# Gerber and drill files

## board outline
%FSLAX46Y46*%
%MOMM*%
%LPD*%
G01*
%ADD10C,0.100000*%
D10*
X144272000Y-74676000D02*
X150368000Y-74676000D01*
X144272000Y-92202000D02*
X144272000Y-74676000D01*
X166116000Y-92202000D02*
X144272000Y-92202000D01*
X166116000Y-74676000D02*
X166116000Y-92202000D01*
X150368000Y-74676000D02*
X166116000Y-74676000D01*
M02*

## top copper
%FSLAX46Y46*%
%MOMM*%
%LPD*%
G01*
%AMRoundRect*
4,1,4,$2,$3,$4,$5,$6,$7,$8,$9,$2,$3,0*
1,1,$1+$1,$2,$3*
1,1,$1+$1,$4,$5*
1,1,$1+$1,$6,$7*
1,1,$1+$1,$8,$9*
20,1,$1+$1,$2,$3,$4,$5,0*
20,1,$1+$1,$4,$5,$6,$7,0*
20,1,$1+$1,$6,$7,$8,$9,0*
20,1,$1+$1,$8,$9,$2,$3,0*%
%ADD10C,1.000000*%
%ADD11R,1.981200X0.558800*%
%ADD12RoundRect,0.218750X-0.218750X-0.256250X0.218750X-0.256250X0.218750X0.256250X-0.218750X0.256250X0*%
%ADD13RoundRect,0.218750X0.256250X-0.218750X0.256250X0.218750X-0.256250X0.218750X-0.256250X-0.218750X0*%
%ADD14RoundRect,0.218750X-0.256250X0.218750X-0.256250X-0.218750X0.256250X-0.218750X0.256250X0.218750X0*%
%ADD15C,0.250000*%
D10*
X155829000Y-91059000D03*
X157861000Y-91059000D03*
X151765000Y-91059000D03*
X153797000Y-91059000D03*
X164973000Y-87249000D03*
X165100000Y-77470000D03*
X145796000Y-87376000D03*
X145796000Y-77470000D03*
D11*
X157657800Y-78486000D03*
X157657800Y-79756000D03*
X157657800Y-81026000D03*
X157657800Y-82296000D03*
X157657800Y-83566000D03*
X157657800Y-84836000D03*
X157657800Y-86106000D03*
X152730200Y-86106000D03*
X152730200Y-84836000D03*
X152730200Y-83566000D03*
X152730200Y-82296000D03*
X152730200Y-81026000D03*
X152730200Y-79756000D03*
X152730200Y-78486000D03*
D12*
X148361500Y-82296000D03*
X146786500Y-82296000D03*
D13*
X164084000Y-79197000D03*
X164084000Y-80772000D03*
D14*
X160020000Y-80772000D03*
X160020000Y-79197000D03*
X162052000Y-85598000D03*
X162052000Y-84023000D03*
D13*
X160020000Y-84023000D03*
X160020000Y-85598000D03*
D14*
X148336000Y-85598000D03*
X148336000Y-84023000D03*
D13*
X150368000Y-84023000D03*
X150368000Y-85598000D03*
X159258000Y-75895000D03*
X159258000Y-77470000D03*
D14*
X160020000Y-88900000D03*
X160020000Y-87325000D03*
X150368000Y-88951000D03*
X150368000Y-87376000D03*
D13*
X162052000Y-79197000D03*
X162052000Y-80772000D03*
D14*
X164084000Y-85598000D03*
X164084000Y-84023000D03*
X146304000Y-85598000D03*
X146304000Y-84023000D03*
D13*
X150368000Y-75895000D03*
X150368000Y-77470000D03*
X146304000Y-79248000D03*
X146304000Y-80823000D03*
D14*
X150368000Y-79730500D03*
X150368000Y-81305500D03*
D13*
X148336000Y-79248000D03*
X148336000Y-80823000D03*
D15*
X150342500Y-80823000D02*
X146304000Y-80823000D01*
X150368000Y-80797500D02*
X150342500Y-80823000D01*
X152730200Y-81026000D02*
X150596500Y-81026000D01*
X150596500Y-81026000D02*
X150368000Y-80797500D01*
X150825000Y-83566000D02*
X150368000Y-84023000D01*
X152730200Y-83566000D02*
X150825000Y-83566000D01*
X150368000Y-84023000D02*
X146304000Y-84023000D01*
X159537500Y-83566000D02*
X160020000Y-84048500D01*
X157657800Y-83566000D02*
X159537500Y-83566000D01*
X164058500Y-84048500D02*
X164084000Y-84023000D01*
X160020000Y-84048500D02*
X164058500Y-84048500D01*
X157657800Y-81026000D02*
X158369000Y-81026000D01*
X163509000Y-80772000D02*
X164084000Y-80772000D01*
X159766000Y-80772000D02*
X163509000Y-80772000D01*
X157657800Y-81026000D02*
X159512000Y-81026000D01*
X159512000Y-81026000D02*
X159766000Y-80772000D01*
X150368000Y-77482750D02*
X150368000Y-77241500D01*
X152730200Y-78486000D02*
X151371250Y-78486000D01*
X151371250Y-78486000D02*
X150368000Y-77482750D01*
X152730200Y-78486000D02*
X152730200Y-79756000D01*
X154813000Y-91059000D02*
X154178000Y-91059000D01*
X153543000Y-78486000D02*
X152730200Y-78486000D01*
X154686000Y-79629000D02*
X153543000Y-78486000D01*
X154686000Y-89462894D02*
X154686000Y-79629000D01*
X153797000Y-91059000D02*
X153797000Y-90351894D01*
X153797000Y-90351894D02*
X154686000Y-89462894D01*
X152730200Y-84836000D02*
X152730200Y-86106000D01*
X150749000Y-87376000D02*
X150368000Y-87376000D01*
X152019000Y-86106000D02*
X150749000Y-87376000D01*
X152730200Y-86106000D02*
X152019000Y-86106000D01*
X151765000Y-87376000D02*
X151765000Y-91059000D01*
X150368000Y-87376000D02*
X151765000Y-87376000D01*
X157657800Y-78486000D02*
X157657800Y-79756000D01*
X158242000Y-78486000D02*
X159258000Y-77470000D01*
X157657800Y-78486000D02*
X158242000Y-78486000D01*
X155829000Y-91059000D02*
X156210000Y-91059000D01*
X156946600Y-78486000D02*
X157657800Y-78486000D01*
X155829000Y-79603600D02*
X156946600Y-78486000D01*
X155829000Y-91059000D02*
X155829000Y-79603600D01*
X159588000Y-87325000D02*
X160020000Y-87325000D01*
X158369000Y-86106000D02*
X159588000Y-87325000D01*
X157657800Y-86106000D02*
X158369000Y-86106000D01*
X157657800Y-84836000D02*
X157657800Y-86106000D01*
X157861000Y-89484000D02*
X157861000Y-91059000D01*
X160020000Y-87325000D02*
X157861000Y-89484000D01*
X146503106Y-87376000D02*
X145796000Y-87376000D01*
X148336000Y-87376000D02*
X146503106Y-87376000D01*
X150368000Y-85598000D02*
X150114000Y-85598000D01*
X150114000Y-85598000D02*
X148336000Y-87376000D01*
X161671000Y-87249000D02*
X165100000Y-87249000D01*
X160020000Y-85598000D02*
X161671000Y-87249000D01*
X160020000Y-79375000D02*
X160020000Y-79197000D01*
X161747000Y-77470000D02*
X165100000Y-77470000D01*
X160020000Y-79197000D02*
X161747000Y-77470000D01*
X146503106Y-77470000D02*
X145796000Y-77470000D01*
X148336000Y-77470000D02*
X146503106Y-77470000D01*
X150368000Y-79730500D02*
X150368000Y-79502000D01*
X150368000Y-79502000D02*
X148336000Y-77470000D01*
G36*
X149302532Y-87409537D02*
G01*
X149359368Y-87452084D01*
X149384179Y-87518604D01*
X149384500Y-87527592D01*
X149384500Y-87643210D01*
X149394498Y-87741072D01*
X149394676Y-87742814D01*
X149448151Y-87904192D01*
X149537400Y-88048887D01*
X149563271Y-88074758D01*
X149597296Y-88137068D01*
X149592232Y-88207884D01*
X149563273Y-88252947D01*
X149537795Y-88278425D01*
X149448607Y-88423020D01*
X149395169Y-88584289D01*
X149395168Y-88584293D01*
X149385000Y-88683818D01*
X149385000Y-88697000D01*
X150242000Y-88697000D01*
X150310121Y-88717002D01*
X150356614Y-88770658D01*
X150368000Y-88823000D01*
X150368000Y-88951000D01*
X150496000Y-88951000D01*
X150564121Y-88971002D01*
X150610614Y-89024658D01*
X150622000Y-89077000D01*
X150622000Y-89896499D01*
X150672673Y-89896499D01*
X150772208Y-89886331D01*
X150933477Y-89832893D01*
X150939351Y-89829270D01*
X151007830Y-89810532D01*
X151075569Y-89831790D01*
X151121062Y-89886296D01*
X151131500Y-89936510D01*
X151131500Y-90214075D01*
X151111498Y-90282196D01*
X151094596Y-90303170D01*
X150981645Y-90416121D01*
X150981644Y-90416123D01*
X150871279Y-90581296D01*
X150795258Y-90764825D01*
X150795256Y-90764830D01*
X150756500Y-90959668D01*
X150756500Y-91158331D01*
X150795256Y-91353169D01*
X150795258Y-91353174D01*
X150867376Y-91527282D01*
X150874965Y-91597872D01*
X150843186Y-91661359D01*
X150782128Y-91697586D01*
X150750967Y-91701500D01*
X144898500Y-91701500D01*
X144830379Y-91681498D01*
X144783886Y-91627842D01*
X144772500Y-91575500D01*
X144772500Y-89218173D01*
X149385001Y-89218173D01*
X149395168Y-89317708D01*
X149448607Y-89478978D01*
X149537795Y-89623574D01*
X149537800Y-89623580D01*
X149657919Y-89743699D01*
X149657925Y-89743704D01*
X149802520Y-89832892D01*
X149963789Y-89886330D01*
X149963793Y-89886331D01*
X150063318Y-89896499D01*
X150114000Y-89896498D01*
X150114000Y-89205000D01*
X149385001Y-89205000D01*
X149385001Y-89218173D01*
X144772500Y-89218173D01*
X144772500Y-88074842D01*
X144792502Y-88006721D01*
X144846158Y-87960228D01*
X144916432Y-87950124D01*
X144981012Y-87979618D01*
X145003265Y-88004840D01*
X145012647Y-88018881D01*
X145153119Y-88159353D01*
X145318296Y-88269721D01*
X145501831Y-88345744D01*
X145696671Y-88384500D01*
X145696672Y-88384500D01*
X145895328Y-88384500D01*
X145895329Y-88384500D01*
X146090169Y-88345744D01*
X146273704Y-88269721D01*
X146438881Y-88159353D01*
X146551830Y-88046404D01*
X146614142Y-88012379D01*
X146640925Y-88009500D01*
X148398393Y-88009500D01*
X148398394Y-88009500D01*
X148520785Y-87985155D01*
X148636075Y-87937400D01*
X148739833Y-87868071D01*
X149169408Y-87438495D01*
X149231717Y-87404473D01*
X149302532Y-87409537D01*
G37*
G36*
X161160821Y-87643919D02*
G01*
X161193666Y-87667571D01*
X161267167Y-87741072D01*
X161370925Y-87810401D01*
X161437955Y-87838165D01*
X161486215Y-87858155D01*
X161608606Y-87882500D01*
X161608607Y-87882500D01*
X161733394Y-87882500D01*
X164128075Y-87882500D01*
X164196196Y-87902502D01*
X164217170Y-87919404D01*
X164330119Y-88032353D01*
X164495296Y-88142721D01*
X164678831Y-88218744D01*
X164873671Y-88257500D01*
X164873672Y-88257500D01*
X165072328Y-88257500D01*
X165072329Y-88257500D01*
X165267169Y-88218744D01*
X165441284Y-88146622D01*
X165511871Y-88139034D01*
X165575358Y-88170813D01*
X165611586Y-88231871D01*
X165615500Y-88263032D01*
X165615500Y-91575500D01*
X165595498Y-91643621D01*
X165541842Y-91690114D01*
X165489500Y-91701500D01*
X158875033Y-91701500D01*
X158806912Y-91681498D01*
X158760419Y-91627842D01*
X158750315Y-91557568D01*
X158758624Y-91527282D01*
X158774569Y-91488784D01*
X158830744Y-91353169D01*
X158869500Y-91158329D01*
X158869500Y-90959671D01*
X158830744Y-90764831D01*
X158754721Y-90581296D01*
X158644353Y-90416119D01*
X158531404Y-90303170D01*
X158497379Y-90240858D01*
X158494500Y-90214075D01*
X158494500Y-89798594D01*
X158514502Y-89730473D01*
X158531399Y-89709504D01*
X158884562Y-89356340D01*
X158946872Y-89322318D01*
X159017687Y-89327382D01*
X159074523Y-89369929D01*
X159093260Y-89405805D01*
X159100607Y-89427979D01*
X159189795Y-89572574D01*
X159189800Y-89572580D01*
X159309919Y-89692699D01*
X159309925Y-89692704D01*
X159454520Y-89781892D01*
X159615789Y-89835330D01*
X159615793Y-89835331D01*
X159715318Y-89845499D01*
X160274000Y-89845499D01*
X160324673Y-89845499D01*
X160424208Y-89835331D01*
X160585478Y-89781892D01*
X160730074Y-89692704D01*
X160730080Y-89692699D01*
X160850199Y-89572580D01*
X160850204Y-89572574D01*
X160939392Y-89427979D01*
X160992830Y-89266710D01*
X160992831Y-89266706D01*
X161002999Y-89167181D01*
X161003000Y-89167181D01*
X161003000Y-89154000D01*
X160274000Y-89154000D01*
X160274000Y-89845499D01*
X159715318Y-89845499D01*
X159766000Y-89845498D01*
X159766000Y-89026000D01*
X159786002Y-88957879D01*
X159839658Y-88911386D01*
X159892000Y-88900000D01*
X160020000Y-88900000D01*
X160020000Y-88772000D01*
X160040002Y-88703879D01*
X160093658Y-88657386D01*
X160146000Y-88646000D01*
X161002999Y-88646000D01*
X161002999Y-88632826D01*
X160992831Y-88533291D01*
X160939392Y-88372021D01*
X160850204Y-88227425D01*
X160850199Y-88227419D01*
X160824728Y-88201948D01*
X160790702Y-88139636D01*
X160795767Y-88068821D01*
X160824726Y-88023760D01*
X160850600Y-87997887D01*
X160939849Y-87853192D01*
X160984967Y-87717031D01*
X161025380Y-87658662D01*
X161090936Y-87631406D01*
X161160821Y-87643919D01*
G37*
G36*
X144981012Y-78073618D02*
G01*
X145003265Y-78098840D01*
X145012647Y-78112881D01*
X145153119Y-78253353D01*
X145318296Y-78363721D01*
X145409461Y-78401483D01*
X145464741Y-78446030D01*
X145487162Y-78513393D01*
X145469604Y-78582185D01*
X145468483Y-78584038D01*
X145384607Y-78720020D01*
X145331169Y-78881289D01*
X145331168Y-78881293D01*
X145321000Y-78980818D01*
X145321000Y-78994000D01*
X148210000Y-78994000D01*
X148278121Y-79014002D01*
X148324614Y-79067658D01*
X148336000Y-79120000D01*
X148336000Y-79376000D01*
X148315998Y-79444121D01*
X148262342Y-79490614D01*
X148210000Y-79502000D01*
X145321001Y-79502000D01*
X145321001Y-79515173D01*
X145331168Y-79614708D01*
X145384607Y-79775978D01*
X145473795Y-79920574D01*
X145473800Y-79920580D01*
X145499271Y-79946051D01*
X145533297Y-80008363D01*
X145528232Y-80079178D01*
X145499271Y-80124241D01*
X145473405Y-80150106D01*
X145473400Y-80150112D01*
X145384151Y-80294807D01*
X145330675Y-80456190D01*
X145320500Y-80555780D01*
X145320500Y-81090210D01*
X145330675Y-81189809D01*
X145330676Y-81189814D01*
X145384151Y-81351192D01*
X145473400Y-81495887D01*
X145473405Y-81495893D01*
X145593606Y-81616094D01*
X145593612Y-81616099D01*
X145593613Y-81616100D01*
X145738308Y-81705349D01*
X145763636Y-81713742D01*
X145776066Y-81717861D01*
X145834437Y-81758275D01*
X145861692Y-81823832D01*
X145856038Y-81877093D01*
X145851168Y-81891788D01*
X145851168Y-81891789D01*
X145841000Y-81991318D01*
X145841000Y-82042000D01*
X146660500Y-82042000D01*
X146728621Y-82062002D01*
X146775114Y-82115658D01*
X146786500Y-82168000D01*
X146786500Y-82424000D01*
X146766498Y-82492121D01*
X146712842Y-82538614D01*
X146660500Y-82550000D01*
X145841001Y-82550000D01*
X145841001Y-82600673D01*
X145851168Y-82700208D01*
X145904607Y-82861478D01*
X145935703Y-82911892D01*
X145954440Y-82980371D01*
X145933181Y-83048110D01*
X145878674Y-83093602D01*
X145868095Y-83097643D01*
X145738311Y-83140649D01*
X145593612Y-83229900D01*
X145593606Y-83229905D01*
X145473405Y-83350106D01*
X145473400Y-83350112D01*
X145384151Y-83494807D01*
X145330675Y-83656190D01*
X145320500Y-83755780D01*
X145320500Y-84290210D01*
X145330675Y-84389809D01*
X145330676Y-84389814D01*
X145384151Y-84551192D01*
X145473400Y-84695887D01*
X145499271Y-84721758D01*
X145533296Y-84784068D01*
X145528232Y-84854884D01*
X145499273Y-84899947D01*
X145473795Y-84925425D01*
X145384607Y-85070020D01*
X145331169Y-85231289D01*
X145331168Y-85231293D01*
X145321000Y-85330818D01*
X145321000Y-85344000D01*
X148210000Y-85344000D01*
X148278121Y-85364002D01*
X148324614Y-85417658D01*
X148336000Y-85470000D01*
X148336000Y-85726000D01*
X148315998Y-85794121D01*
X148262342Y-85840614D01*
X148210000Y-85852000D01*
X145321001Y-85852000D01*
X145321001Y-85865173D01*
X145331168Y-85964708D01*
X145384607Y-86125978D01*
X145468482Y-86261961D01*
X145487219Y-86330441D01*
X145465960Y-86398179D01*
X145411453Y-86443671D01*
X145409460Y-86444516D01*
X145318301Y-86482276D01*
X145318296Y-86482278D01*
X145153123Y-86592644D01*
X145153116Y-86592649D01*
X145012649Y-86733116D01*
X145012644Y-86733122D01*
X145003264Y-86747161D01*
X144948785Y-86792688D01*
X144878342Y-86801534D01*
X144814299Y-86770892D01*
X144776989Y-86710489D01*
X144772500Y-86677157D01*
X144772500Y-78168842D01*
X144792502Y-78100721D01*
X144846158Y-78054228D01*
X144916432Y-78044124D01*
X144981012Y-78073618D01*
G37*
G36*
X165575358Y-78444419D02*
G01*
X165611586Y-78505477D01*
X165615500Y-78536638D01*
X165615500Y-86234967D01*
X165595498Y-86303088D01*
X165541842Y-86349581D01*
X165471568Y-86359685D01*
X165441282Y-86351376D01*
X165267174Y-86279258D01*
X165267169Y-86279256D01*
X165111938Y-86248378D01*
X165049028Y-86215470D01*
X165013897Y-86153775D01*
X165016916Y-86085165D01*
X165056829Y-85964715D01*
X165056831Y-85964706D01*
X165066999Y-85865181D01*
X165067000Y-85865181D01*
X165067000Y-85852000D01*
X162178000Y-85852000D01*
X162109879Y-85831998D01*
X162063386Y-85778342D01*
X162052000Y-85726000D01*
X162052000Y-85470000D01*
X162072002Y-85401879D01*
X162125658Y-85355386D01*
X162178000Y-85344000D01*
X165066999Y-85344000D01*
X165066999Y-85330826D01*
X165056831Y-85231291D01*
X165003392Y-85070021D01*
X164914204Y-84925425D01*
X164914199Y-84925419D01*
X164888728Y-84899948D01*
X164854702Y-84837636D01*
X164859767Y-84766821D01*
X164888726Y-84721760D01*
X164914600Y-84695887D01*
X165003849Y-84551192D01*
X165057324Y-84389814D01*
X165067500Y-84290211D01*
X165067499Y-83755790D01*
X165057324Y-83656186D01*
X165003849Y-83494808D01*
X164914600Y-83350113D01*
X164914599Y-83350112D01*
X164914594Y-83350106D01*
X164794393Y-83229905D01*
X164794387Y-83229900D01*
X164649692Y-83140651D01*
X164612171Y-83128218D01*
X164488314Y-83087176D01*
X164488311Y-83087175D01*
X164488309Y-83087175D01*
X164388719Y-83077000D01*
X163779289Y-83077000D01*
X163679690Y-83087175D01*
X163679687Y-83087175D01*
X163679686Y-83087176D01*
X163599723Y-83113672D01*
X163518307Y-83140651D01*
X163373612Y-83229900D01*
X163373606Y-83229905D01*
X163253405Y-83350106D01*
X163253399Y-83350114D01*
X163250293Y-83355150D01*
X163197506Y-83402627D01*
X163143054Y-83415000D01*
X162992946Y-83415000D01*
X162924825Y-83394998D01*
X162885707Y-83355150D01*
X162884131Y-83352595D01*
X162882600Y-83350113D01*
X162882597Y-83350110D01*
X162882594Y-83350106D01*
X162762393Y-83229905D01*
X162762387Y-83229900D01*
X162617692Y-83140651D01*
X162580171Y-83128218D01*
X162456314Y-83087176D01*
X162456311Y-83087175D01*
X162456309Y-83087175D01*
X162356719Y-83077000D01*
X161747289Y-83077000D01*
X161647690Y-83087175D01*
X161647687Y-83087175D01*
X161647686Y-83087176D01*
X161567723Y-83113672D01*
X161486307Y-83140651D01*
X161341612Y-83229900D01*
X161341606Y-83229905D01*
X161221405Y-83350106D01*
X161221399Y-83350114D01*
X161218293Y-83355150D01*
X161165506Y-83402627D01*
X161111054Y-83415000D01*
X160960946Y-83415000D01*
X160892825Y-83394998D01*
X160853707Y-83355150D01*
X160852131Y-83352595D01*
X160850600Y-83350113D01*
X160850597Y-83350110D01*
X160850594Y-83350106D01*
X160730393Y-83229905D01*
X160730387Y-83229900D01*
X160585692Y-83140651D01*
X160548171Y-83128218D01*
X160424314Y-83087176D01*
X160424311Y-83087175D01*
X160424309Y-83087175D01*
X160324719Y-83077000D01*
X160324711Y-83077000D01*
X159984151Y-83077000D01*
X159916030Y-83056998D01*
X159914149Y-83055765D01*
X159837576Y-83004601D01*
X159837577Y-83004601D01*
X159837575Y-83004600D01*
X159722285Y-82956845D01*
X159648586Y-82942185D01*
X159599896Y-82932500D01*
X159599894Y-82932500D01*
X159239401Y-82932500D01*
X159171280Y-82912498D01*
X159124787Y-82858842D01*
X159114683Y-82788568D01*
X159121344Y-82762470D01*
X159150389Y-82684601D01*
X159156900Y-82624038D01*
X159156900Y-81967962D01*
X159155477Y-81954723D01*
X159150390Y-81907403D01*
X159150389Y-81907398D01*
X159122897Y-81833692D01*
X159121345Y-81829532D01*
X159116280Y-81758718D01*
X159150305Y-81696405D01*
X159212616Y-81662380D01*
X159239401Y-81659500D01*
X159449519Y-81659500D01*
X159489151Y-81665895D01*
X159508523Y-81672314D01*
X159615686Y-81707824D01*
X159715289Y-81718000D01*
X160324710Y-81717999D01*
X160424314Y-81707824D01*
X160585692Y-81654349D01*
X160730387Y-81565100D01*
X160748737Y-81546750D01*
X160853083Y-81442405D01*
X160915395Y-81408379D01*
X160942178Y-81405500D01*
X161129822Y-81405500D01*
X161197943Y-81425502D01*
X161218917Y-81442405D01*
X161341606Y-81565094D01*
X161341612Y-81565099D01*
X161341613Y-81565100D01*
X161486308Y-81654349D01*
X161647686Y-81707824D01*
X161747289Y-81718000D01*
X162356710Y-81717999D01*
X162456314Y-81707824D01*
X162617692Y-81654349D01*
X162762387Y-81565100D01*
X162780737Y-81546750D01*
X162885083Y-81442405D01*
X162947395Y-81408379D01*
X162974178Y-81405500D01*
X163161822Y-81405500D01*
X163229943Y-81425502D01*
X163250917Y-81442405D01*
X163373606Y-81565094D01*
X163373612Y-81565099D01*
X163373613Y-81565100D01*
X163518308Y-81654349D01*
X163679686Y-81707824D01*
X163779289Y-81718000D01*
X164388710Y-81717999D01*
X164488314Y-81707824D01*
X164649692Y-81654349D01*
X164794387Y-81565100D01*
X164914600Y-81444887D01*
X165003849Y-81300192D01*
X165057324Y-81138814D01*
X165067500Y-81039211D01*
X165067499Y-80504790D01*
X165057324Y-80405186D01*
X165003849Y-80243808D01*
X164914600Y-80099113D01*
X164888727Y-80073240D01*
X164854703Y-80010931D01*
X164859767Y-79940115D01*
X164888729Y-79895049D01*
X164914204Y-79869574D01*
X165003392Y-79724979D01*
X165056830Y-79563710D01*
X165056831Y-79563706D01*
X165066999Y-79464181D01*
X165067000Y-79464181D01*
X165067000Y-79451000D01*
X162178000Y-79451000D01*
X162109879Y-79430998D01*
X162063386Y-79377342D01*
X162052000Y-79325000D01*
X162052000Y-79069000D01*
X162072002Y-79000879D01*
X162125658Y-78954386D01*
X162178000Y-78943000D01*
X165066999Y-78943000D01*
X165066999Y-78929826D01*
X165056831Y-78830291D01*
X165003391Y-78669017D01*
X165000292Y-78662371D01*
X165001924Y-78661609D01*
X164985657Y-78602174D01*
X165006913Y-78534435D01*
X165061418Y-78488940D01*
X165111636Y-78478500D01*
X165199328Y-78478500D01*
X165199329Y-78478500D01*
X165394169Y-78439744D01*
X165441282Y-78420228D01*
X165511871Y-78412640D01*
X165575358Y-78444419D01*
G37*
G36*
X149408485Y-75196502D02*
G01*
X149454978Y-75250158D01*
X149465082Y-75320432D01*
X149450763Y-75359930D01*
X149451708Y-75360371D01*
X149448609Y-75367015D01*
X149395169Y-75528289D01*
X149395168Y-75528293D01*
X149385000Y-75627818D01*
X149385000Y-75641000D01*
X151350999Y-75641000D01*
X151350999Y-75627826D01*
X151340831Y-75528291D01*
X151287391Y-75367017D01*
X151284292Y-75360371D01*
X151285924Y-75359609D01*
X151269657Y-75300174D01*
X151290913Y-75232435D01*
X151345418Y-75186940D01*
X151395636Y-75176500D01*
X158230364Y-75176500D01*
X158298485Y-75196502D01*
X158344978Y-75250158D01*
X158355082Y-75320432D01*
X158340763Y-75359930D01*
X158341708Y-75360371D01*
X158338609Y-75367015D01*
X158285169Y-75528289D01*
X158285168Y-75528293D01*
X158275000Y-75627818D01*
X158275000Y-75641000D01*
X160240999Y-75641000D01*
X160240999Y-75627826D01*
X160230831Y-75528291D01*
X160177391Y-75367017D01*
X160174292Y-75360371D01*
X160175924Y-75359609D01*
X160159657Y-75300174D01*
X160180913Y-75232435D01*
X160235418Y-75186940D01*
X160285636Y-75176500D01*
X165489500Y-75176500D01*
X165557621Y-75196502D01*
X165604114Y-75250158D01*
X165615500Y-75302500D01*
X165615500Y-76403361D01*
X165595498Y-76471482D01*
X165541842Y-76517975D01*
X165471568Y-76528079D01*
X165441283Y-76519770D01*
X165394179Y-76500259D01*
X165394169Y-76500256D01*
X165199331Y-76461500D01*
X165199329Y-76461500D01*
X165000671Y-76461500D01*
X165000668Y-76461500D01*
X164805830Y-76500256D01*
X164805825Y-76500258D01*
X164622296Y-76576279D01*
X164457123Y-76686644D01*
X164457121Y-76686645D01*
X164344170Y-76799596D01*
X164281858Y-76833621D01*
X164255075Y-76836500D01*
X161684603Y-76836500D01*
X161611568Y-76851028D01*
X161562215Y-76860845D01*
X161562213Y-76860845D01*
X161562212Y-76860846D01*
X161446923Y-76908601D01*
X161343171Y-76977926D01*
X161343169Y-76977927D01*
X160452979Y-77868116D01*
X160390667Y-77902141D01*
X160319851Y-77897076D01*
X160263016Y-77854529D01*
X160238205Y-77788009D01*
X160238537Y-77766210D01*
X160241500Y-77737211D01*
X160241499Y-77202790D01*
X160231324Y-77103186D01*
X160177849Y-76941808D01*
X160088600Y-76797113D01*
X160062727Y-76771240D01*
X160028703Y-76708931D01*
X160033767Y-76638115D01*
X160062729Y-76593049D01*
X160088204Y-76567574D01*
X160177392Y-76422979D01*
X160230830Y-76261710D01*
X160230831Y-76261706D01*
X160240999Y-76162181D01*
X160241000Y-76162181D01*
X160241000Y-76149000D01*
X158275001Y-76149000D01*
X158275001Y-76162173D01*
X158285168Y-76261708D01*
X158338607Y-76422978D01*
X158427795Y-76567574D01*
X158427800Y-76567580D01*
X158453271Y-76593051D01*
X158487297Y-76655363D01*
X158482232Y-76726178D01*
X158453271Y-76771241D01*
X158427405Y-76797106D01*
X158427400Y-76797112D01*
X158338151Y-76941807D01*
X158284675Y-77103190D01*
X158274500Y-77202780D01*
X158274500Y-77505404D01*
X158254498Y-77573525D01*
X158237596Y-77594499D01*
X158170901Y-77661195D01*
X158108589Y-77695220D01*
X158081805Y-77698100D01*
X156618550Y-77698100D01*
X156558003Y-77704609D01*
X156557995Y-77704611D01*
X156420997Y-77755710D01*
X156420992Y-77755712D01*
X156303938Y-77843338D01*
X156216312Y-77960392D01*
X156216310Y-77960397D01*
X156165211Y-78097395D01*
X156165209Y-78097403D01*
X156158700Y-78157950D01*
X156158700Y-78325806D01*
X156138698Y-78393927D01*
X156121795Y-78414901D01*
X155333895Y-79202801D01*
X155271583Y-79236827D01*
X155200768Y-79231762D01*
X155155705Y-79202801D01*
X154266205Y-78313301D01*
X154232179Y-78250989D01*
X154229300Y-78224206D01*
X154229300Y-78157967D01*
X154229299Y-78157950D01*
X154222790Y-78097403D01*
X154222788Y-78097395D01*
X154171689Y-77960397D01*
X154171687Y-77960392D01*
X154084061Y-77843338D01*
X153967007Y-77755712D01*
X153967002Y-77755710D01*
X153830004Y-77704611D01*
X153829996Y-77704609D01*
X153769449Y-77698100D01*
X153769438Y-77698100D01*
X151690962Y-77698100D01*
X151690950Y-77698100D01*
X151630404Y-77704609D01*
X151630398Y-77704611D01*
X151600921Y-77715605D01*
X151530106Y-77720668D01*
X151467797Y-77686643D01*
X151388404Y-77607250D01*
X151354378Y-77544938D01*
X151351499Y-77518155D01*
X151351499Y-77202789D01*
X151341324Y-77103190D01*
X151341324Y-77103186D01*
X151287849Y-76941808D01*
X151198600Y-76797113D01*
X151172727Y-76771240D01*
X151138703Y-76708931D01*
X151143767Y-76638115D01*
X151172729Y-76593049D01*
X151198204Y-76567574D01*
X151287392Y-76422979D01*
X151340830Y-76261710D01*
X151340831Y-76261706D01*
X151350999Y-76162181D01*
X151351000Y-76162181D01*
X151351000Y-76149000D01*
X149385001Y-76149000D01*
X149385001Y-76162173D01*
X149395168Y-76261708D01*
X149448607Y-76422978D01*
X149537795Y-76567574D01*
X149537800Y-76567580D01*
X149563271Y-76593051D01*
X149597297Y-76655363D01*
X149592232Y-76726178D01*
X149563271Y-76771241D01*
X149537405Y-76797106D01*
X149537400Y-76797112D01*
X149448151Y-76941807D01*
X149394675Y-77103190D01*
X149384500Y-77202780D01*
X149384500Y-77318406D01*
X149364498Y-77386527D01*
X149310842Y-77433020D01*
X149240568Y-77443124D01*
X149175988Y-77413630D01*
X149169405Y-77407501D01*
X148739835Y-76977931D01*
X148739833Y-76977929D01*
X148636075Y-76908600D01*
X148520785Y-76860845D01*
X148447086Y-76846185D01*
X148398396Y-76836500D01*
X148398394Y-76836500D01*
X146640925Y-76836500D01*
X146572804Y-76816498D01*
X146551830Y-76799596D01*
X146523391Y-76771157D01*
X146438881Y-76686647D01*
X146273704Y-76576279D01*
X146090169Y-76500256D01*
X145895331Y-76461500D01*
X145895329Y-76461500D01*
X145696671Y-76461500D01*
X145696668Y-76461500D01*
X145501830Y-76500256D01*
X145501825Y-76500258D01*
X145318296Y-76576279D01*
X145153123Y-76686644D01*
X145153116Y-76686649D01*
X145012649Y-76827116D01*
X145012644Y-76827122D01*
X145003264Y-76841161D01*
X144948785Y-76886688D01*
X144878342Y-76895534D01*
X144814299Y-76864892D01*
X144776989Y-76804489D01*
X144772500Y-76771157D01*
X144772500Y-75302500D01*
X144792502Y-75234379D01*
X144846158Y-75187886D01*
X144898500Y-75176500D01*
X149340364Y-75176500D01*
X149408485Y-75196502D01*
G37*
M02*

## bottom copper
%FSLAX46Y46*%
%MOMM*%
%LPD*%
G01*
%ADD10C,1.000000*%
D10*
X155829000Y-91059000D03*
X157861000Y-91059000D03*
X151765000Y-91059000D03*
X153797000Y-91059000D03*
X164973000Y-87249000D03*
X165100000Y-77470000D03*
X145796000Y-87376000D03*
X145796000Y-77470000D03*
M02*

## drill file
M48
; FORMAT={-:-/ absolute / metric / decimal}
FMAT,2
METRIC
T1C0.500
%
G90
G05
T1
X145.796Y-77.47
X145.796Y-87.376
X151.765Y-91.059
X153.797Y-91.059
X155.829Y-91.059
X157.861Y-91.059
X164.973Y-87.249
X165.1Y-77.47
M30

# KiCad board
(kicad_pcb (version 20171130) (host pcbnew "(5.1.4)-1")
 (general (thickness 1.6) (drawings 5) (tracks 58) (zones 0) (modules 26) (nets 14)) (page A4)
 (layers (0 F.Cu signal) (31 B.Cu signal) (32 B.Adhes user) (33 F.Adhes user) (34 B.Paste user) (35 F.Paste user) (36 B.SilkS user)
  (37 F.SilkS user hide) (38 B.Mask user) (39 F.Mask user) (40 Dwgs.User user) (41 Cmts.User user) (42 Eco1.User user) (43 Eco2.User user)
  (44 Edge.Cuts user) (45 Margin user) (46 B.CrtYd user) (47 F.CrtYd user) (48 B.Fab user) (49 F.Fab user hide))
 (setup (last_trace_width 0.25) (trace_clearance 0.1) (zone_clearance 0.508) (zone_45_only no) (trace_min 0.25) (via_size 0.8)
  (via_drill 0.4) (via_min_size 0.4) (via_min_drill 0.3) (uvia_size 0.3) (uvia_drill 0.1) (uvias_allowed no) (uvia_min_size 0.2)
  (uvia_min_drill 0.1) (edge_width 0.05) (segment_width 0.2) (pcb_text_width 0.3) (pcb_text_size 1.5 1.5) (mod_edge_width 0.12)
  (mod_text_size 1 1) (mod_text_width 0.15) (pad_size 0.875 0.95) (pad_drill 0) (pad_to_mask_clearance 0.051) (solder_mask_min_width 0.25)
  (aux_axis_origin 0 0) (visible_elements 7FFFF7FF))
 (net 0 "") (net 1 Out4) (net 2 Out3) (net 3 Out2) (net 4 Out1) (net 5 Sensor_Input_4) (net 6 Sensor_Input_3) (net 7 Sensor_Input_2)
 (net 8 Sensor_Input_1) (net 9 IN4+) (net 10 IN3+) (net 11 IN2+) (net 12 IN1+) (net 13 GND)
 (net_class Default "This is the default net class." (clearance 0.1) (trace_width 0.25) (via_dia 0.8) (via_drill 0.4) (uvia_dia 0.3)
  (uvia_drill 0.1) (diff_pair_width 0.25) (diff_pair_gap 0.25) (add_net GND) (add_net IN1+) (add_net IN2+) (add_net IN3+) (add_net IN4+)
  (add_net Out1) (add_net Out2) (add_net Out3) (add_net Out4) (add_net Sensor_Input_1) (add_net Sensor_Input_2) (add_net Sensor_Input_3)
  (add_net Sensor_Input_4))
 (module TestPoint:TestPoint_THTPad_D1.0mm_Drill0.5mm (layer F.Cu) (at 155.829 91.059)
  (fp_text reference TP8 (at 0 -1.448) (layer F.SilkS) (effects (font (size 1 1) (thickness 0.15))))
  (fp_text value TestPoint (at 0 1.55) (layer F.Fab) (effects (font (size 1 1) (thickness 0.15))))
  (pad 1 thru_hole circle (at 0 0) (size 1 1) (drill 0.5) (layers *.Cu *.Mask) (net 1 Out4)))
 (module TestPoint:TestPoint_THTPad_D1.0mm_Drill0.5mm (layer F.Cu) (at 157.861 91.059)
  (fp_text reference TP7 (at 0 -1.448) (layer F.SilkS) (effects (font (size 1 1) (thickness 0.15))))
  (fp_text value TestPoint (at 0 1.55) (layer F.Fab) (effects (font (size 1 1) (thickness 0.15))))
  (pad 1 thru_hole circle (at 0 0) (size 1 1) (drill 0.5) (layers *.Cu *.Mask) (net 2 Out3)))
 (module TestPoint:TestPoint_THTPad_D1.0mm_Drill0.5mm (layer F.Cu) (at 151.765 91.059)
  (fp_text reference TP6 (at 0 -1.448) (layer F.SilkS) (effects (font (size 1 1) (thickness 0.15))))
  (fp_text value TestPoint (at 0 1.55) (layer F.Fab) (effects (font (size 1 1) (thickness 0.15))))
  (pad 1 thru_hole circle (at 0 0) (size 1 1) (drill 0.5) (layers *.Cu *.Mask) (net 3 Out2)))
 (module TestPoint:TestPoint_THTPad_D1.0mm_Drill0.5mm (layer F.Cu) (at 153.797 91.059)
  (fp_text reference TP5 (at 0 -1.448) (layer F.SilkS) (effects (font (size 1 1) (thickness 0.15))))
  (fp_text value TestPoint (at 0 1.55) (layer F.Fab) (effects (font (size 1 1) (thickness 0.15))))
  (pad 1 thru_hole circle (at 0 0) (size 1 1) (drill 0.5) (layers *.Cu *.Mask) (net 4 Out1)))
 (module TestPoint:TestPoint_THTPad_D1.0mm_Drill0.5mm (layer F.Cu) (at 164.973 87.249)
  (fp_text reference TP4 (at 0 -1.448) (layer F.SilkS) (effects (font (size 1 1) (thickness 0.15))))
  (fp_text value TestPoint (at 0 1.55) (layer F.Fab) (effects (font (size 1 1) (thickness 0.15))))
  (pad 1 thru_hole circle (at 0 0) (size 1 1) (drill 0.5) (layers *.Cu *.Mask) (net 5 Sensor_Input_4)))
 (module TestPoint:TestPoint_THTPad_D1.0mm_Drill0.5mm (layer F.Cu) (at 165.1 77.47)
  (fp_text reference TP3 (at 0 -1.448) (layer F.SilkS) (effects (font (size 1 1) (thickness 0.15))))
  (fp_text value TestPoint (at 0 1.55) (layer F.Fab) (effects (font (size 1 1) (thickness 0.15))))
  (pad 1 thru_hole circle (at 0 0) (size 1 1) (drill 0.5) (layers *.Cu *.Mask) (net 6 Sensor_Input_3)))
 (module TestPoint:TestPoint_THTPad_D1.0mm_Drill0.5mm (layer F.Cu) (at 145.796 87.376)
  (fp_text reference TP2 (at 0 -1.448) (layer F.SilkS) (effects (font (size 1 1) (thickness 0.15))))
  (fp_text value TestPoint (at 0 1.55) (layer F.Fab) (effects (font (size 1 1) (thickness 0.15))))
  (pad 1 thru_hole circle (at 0 0) (size 1 1) (drill 0.5) (layers *.Cu *.Mask) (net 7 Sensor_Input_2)))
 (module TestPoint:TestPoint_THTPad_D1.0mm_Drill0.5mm (layer F.Cu) (at 145.796 77.47)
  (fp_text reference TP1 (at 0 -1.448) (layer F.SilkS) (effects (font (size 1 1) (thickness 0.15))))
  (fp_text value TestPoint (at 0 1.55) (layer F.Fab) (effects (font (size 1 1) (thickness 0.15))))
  (pad 1 thru_hole circle (at 0 0) (size 1 1) (drill 0.5) (layers *.Cu *.Mask) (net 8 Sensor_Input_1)))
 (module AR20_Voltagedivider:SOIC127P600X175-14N (layer F.Cu) (at 155.194 82.296)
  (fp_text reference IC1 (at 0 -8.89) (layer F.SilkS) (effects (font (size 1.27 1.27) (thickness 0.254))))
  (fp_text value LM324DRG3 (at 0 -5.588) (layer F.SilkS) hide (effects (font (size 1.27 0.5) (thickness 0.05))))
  (pad 14 smd rect (at 2.4638 -3.81 90) (size 0.5588 1.9812) (layers F.Cu F.Paste F.Mask) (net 1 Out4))
  (pad 13 smd rect (at 2.4638 -2.54 90) (size 0.5588 1.9812) (layers F.Cu F.Paste F.Mask) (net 1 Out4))
  (pad 12 smd rect (at 2.4638 -1.27 90) (size 0.5588 1.9812) (layers F.Cu F.Paste F.Mask) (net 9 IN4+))
  (pad 11 smd rect (at 2.4638 0 90) (size 0.5588 1.9812) (layers F.Cu F.Paste F.Mask))
  (pad 10 smd rect (at 2.4638 1.27 90) (size 0.5588 1.9812) (layers F.Cu F.Paste F.Mask) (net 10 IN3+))
  (pad 9 smd rect (at 2.4638 2.54 90) (size 0.5588 1.9812) (layers F.Cu F.Paste F.Mask) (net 2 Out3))
  (pad 8 smd rect (at 2.4638 3.81 90) (size 0.5588 1.9812) (layers F.Cu F.Paste F.Mask) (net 2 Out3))
  (pad 7 smd rect (at -2.4638 3.81 90) (size 0.5588 1.9812) (layers F.Cu F.Paste F.Mask) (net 3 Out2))
  (pad 6 smd rect (at -2.4638 2.54 90) (size 0.5588 1.9812) (layers F.Cu F.Paste F.Mask) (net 3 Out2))
  (pad 5 smd rect (at -2.4638 1.27 90) (size 0.5588 1.9812) (layers F.Cu F.Paste F.Mask) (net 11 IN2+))
  (pad 4 smd rect (at -2.4638 0 90) (size 0.5588 1.9812) (layers F.Cu F.Paste F.Mask))
  (pad 3 smd rect (at -2.4638 -1.27 90) (size 0.5588 1.9812) (layers F.Cu F.Paste F.Mask) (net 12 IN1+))
  (pad 2 smd rect (at -2.4638 -2.54 90) (size 0.5588 1.9812) (layers F.Cu F.Paste F.Mask) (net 4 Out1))
  (pad 1 smd rect (at -2.4638 -3.81 90) (size 0.5588 1.9812) (layers F.Cu F.Paste F.Mask) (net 4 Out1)))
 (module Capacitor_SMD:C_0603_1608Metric (layer F.Cu) (at 147.574 82.296)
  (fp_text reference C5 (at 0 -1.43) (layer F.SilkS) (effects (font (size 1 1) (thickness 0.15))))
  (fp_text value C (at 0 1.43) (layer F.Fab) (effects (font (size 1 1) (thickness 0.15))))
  (pad 2 smd roundrect (at 0.7875 0) (size 0.875 0.95) (layers F.Cu F.Paste F.Mask) (roundrect_rratio 0.25))
  (pad 1 smd roundrect (at -0.7875 0) (size 0.875 0.95) (layers F.Cu F.Paste F.Mask) (roundrect_rratio 0.25) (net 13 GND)))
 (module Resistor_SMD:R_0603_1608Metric (layer F.Cu) (at 164.084 79.9845 90)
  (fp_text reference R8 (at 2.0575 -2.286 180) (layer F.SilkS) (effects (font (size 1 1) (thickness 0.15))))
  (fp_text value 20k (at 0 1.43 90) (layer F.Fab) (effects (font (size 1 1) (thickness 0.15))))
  (pad 2 smd roundrect (at 0.7875 0 90) (size 0.875 0.95) (layers F.Cu F.Paste F.Mask) (roundrect_rratio 0.25) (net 13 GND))
  (pad 1 smd roundrect (at -0.7875 0 90) (size 0.875 0.95) (layers F.Cu F.Paste F.Mask) (roundrect_rratio 0.25) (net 9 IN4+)))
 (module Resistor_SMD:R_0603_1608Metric (layer F.Cu) (at 160.02 79.9845 270)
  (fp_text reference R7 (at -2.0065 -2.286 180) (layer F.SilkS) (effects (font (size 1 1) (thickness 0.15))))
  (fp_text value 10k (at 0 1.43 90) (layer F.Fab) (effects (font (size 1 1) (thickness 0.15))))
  (pad 2 smd roundrect (at 0.7875 0 270) (size 0.875 0.95) (layers F.Cu F.Paste F.Mask) (roundrect_rratio 0.25) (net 9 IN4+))
  (pad 1 smd roundrect (at -0.7875 0 270) (size 0.875 0.95) (layers F.Cu F.Paste F.Mask) (roundrect_rratio 0.25) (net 6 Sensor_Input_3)))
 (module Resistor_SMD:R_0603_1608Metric (layer F.Cu) (at 162.052 84.8105 270)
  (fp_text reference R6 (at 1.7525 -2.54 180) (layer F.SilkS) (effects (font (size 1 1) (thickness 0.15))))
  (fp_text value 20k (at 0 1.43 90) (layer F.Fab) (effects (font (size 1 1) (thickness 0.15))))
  (pad 2 smd roundrect (at 0.7875 0 270) (size 0.875 0.95) (layers F.Cu F.Paste F.Mask) (roundrect_rratio 0.25) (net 13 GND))
  (pad 1 smd roundrect (at -0.7875 0 270) (size 0.875 0.95) (layers F.Cu F.Paste F.Mask) (roundrect_rratio 0.25) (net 10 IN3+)))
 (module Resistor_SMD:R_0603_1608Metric (layer F.Cu) (at 160.02 84.8105 90)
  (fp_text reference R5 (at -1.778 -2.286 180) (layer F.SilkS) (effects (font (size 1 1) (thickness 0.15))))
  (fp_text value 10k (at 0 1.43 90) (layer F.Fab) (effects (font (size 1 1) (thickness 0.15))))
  (pad 2 smd roundrect (at 0.7875 0 90) (size 0.875 0.95) (layers F.Cu F.Paste F.Mask) (roundrect_rratio 0.25) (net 10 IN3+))
  (pad 1 smd roundrect (at -0.7875 0 90) (size 0.875 0.95) (layers F.Cu F.Paste F.Mask) (roundrect_rratio 0.25) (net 5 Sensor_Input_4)))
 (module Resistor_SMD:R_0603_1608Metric (layer F.Cu) (at 148.336 84.8105 270)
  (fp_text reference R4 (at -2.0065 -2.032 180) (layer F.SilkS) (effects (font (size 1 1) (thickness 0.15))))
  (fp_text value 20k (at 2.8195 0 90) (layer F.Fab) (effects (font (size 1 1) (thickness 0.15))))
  (pad 2 smd roundrect (at 0.7875 0 270) (size 0.875 0.95) (layers F.Cu F.Paste F.Mask) (roundrect_rratio 0.25) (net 13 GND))
  (pad 1 smd roundrect (at -0.7875 0 270) (size 0.875 0.95) (layers F.Cu F.Paste F.Mask) (roundrect_rratio 0.25) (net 11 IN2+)))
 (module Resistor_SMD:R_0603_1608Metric (layer F.Cu) (at 150.368 84.8105 90)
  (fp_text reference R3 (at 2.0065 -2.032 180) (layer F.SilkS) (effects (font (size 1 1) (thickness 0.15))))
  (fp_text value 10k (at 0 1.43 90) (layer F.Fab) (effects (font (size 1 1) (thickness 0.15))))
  (pad 2 smd roundrect (at 0.7875 0 90) (size 0.875 0.95) (layers F.Cu F.Paste F.Mask) (roundrect_rratio 0.25) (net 11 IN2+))
  (pad 1 smd roundrect (at -0.7875 0 90) (size 0.875 0.95) (layers F.Cu F.Paste F.Mask) (roundrect_rratio 0.25) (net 7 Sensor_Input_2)))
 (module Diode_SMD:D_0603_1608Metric (layer F.Cu) (at 159.258 76.6825 90)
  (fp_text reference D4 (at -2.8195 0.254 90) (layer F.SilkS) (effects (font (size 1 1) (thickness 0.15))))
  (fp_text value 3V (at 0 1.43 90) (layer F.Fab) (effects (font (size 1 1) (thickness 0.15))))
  (pad 2 smd roundrect (at 0.7875 0 90) (size 0.875 0.95) (layers F.Cu F.Paste F.Mask) (roundrect_rratio 0.25) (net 13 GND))
  (pad 1 smd roundrect (at -0.7875 0 90) (size 0.875 0.95) (layers F.Cu F.Paste F.Mask) (roundrect_rratio 0.25) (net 1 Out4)))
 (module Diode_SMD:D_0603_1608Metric (layer F.Cu) (at 160.02 88.1125 270)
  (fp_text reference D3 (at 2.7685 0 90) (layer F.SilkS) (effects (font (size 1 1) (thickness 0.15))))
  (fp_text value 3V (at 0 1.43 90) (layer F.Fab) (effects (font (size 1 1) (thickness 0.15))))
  (pad 2 smd roundrect (at 0.7875 0 270) (size 0.875 0.95) (layers F.Cu F.Paste F.Mask) (roundrect_rratio 0.25) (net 13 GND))
  (pad 1 smd roundrect (at -0.7875 0 270) (size 0.875 0.95) (layers F.Cu F.Paste F.Mask) (roundrect_rratio 0.25) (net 2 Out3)))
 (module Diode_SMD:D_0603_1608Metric (layer F.Cu) (at 150.368 88.1635 270)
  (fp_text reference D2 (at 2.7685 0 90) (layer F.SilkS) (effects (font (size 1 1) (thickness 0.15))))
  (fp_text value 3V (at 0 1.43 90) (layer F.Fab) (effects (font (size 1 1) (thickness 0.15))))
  (pad 2 smd roundrect (at 0.7875 0 270) (size 0.875 0.95) (layers F.Cu F.Paste F.Mask) (roundrect_rratio 0.25) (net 13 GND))
  (pad 1 smd roundrect (at -0.7875 0 270) (size 0.875 0.95) (layers F.Cu F.Paste F.Mask) (roundrect_rratio 0.25) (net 3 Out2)))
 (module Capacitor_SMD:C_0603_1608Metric (layer F.Cu) (at 162.052 79.9845 90)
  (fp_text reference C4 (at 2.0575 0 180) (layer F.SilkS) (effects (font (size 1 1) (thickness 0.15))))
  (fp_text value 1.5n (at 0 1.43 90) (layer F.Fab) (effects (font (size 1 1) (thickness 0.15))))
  (pad 2 smd roundrect (at 0.7875 0 90) (size 0.875 0.95) (layers F.Cu F.Paste F.Mask) (roundrect_rratio 0.25) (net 13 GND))
  (pad 1 smd roundrect (at -0.7875 0 90) (size 0.875 0.95) (layers F.Cu F.Paste F.Mask) (roundrect_rratio 0.25) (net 9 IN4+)))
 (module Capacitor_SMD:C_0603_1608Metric (layer F.Cu) (at 164.084 84.8105 270)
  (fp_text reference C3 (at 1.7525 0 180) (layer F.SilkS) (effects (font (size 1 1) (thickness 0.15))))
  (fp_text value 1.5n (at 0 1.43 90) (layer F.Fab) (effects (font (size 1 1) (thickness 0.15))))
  (pad 2 smd roundrect (at 0.7875 0 270) (size 0.875 0.95) (layers F.Cu F.Paste F.Mask) (roundrect_rratio 0.25) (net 13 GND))
  (pad 1 smd roundrect (at -0.7875 0 270) (size 0.875 0.95) (layers F.Cu F.Paste F.Mask) (roundrect_rratio 0.25) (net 10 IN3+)))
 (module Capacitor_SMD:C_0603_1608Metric (layer F.Cu) (at 146.304 84.8105 270)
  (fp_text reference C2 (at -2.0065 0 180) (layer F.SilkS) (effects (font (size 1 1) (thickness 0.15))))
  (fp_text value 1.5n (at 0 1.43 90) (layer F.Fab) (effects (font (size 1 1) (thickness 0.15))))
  (pad 2 smd roundrect (at 0.7875 0 270) (size 0.875 0.95) (layers F.Cu F.Paste F.Mask) (roundrect_rratio 0.25) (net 13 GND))
  (pad 1 smd roundrect (at -0.7875 0 270) (size 0.875 0.95) (layers F.Cu F.Paste F.Mask) (roundrect_rratio 0.25) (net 11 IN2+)))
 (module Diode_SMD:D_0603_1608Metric (layer F.Cu) (at 150.368 76.6825 90)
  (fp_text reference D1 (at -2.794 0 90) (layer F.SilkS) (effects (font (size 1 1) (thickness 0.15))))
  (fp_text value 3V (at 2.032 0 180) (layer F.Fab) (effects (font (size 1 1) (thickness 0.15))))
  (pad 2 smd roundrect (at 0.7875 0 90) (size 0.875 0.95) (layers F.Cu F.Paste F.Mask) (roundrect_rratio 0.25) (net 13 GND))
  (pad 1 smd roundrect (at -0.7875 0 90) (size 0.875 0.95) (layers F.Cu F.Paste F.Mask) (roundrect_rratio 0.25) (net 4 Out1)))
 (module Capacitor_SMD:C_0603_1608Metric (layer F.Cu) (at 146.304 80.0355 90)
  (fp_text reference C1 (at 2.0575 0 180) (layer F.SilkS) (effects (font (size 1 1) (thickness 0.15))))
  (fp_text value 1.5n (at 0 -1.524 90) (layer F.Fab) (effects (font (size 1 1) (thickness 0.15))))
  (pad 2 smd roundrect (at 0.7875 0 90) (size 0.875 0.95) (layers F.Cu F.Paste F.Mask) (roundrect_rratio 0.25) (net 13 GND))
  (pad 1 smd roundrect (at -0.7875 0 90) (size 0.875 0.95) (layers F.Cu F.Paste F.Mask) (roundrect_rratio 0.25) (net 12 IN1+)))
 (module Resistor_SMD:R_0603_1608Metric (layer F.Cu) (at 150.368 80.518 270)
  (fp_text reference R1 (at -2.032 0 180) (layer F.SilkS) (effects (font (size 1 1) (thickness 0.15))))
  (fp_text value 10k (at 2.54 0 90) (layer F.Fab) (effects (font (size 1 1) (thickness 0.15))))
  (pad 1 smd roundrect (at -0.7875 0 270) (size 0.875 0.95) (layers F.Cu F.Paste F.Mask) (roundrect_rratio 0.25) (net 8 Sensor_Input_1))
  (pad 2 smd roundrect (at 0.7875 0 270) (size 0.875 0.95) (layers F.Cu F.Paste F.Mask) (roundrect_rratio 0.25) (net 12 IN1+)))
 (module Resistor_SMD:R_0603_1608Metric (layer F.Cu) (at 148.336 80.0355 90)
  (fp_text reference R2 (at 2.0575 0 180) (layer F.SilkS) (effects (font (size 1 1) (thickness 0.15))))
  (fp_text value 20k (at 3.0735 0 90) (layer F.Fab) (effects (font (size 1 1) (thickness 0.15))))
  (pad 2 smd roundrect (at 0.7875 0 90) (size 0.875 0.95) (layers F.Cu F.Paste F.Mask) (roundrect_rratio 0.25) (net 13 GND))
  (pad 1 smd roundrect (at -0.7875 0 90) (size 0.875 0.95) (layers F.Cu F.Paste F.Mask) (roundrect_rratio 0.25) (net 12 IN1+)))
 (gr_line (start 144.272 74.676) (end 150.368 74.676) (layer Edge.Cuts) (width 0.1))
 (gr_line (start 144.272 92.202) (end 144.272 74.676) (layer Edge.Cuts) (width 0.1))
 (gr_line (start 166.116 92.202) (end 144.272 92.202) (layer Edge.Cuts) (width 0.1))
 (gr_line (start 166.116 74.676) (end 166.116 92.202) (layer Edge.Cuts) (width 0.1))
 (gr_line (start 150.368 74.676) (end 166.116 74.676) (layer Edge.Cuts) (width 0.1))
 (segment (start 150.3425 80.823) (end 146.304 80.823) (width 0.25) (layer F.Cu) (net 12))
 (segment (start 150.368 80.7975) (end 150.3425 80.823) (width 0.25) (layer F.Cu) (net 12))
 (segment (start 152.7302 81.026) (end 150.5965 81.026) (width 0.25) (layer F.Cu) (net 12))
 (segment (start 150.5965 81.026) (end 150.368 80.7975) (width 0.25) (layer F.Cu) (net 12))
 (segment (start 150.825 83.566) (end 150.368 84.023) (width 0.25) (layer F.Cu) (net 11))
 (segment (start 152.7302 83.566) (end 150.825 83.566) (width 0.25) (layer F.Cu) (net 11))
 (segment (start 150.368 84.023) (end 146.304 84.023) (width 0.25) (layer F.Cu) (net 11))
 (segment (start 159.5375 83.566) (end 160.02 84.0485) (width 0.25) (layer F.Cu) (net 10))
 (segment (start 157.6578 83.566) (end 159.5375 83.566) (width 0.25) (layer F.Cu) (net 10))
 (segment (start 164.0585 84.0485) (end 164.084 84.023) (width 0.25) (layer F.Cu) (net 10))
 (segment (start 160.02 84.0485) (end 164.0585 84.0485) (width 0.25) (layer F.Cu) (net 10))
 (segment (start 157.6578 81.026) (end 158.369 81.026) (width 0.25) (layer F.Cu) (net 9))
 (segment (start 163.509 80.772) (end 164.084 80.772) (width 0.25) (layer F.Cu) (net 9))
 (segment (start 159.766 80.772) (end 163.509 80.772) (width 0.25) (layer F.Cu) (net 9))
 (segment (start 157.6578 81.026) (end 159.512 81.026) (width 0.25) (layer F.Cu) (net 9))
 (segment (start 159.512 81.026) (end 159.766 80.772) (width 0.25) (layer F.Cu) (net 9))
 (segment (start 150.368 77.48275) (end 150.368 77.2415) (width 0.25) (layer F.Cu) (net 4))
 (segment (start 152.7302 78.486) (end 151.37125 78.486) (width 0.25) (layer F.Cu) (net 4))
 (segment (start 151.37125 78.486) (end 150.368 77.48275) (width 0.25) (layer F.Cu) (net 4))
 (segment (start 152.7302 78.486) (end 152.7302 79.756) (width 0.25) (layer F.Cu) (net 4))
 (segment (start 154.813 91.059) (end 154.178 91.059) (width 0.25) (layer F.Cu) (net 4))
 (segment (start 153.543 78.486) (end 152.7302 78.486) (width 0.25) (layer F.Cu) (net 4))
 (segment (start 154.686 79.629) (end 153.543 78.486) (width 0.25) (layer F.Cu) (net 4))
 (segment (start 154.686 89.462894) (end 154.686 79.629) (width 0.25) (layer F.Cu) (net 4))
 (segment (start 153.797 91.059) (end 153.797 90.351894) (width 0.25) (layer F.Cu) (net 4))
 (segment (start 153.797 90.351894) (end 154.686 89.462894) (width 0.25) (layer F.Cu) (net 4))
 (segment (start 152.7302 84.836) (end 152.7302 86.106) (width 0.25) (layer F.Cu) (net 3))
 (segment (start 150.749 87.376) (end 150.368 87.376) (width 0.25) (layer F.Cu) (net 3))
 (segment (start 152.019 86.106) (end 150.749 87.376) (width 0.25) (layer F.Cu) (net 3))
 (segment (start 152.7302 86.106) (end 152.019 86.106) (width 0.25) (layer F.Cu) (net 3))
 (segment (start 151.765 87.376) (end 151.765 91.059) (width 0.25) (layer F.Cu) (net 3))
 (segment (start 150.368 87.376) (end 151.765 87.376) (width 0.25) (layer F.Cu) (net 3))
 (segment (start 157.6578 78.486) (end 157.6578 79.756) (width 0.25) (layer F.Cu) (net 1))
 (segment (start 158.242 78.486) (end 159.258 77.47) (width 0.25) (layer F.Cu) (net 1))
 (segment (start 157.6578 78.486) (end 158.242 78.486) (width 0.25) (layer F.Cu) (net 1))
 (segment (start 155.829 91.059) (end 156.21 91.059) (width 0.25) (layer F.Cu) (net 1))
 (segment (start 156.9466 78.486) (end 157.6578 78.486) (width 0.25) (layer F.Cu) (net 1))
 (segment (start 155.829 79.6036) (end 156.9466 78.486) (width 0.25) (layer F.Cu) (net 1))
 (segment (start 155.829 91.059) (end 155.829 79.6036) (width 0.25) (layer F.Cu) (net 1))
 (segment (start 159.588 87.325) (end 160.02 87.325) (width 0.25) (layer F.Cu) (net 2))
 (segment (start 158.369 86.106) (end 159.588 87.325) (width 0.25) (layer F.Cu) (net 2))
 (segment (start 157.6578 86.106) (end 158.369 86.106) (width 0.25) (layer F.Cu) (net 2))
 (segment (start 157.6578 84.836) (end 157.6578 86.106) (width 0.25) (layer F.Cu) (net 2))
 (segment (start 157.861 89.484) (end 157.861 91.059) (width 0.25) (layer F.Cu) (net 2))
 (segment (start 160.02 87.325) (end 157.861 89.484) (width 0.25) (layer F.Cu) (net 2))
 (segment (start 146.503106 87.376) (end 145.796 87.376) (width 0.25) (layer F.Cu) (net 7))
 (segment (start 148.336 87.376) (end 146.503106 87.376) (width 0.25) (layer F.Cu) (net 7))
 (segment (start 150.368 85.598) (end 150.114 85.598) (width 0.25) (layer F.Cu) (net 7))
 (segment (start 150.114 85.598) (end 148.336 87.376) (width 0.25) (layer F.Cu) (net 7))
 (segment (start 161.671 87.249) (end 165.1 87.249) (width 0.25) (layer F.Cu) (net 5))
 (segment (start 160.02 85.598) (end 161.671 87.249) (width 0.25) (layer F.Cu) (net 5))
 (segment (start 160.02 79.375) (end 160.02 79.197) (width 0.25) (layer F.Cu) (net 6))
 (segment (start 161.747 77.47) (end 165.1 77.47) (width 0.25) (layer F.Cu) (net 6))
 (segment (start 160.02 79.197) (end 161.747 77.47) (width 0.25) (layer F.Cu) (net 6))
 (segment (start 146.503106 77.47) (end 145.796 77.47) (width 0.25) (layer F.Cu) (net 8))
 (segment (start 148.336 77.47) (end 146.503106 77.47) (width 0.25) (layer F.Cu) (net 8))
 (segment (start 150.368 79.7305) (end 150.368 79.502) (width 0.25) (layer F.Cu) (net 8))
 (segment (start 150.368 79.502) (end 148.336 77.47) (width 0.25) (layer F.Cu) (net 8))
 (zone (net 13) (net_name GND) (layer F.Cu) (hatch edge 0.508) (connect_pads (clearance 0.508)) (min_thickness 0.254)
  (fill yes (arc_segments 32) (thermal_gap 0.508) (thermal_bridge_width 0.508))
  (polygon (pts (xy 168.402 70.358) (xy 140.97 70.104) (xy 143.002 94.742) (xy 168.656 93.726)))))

